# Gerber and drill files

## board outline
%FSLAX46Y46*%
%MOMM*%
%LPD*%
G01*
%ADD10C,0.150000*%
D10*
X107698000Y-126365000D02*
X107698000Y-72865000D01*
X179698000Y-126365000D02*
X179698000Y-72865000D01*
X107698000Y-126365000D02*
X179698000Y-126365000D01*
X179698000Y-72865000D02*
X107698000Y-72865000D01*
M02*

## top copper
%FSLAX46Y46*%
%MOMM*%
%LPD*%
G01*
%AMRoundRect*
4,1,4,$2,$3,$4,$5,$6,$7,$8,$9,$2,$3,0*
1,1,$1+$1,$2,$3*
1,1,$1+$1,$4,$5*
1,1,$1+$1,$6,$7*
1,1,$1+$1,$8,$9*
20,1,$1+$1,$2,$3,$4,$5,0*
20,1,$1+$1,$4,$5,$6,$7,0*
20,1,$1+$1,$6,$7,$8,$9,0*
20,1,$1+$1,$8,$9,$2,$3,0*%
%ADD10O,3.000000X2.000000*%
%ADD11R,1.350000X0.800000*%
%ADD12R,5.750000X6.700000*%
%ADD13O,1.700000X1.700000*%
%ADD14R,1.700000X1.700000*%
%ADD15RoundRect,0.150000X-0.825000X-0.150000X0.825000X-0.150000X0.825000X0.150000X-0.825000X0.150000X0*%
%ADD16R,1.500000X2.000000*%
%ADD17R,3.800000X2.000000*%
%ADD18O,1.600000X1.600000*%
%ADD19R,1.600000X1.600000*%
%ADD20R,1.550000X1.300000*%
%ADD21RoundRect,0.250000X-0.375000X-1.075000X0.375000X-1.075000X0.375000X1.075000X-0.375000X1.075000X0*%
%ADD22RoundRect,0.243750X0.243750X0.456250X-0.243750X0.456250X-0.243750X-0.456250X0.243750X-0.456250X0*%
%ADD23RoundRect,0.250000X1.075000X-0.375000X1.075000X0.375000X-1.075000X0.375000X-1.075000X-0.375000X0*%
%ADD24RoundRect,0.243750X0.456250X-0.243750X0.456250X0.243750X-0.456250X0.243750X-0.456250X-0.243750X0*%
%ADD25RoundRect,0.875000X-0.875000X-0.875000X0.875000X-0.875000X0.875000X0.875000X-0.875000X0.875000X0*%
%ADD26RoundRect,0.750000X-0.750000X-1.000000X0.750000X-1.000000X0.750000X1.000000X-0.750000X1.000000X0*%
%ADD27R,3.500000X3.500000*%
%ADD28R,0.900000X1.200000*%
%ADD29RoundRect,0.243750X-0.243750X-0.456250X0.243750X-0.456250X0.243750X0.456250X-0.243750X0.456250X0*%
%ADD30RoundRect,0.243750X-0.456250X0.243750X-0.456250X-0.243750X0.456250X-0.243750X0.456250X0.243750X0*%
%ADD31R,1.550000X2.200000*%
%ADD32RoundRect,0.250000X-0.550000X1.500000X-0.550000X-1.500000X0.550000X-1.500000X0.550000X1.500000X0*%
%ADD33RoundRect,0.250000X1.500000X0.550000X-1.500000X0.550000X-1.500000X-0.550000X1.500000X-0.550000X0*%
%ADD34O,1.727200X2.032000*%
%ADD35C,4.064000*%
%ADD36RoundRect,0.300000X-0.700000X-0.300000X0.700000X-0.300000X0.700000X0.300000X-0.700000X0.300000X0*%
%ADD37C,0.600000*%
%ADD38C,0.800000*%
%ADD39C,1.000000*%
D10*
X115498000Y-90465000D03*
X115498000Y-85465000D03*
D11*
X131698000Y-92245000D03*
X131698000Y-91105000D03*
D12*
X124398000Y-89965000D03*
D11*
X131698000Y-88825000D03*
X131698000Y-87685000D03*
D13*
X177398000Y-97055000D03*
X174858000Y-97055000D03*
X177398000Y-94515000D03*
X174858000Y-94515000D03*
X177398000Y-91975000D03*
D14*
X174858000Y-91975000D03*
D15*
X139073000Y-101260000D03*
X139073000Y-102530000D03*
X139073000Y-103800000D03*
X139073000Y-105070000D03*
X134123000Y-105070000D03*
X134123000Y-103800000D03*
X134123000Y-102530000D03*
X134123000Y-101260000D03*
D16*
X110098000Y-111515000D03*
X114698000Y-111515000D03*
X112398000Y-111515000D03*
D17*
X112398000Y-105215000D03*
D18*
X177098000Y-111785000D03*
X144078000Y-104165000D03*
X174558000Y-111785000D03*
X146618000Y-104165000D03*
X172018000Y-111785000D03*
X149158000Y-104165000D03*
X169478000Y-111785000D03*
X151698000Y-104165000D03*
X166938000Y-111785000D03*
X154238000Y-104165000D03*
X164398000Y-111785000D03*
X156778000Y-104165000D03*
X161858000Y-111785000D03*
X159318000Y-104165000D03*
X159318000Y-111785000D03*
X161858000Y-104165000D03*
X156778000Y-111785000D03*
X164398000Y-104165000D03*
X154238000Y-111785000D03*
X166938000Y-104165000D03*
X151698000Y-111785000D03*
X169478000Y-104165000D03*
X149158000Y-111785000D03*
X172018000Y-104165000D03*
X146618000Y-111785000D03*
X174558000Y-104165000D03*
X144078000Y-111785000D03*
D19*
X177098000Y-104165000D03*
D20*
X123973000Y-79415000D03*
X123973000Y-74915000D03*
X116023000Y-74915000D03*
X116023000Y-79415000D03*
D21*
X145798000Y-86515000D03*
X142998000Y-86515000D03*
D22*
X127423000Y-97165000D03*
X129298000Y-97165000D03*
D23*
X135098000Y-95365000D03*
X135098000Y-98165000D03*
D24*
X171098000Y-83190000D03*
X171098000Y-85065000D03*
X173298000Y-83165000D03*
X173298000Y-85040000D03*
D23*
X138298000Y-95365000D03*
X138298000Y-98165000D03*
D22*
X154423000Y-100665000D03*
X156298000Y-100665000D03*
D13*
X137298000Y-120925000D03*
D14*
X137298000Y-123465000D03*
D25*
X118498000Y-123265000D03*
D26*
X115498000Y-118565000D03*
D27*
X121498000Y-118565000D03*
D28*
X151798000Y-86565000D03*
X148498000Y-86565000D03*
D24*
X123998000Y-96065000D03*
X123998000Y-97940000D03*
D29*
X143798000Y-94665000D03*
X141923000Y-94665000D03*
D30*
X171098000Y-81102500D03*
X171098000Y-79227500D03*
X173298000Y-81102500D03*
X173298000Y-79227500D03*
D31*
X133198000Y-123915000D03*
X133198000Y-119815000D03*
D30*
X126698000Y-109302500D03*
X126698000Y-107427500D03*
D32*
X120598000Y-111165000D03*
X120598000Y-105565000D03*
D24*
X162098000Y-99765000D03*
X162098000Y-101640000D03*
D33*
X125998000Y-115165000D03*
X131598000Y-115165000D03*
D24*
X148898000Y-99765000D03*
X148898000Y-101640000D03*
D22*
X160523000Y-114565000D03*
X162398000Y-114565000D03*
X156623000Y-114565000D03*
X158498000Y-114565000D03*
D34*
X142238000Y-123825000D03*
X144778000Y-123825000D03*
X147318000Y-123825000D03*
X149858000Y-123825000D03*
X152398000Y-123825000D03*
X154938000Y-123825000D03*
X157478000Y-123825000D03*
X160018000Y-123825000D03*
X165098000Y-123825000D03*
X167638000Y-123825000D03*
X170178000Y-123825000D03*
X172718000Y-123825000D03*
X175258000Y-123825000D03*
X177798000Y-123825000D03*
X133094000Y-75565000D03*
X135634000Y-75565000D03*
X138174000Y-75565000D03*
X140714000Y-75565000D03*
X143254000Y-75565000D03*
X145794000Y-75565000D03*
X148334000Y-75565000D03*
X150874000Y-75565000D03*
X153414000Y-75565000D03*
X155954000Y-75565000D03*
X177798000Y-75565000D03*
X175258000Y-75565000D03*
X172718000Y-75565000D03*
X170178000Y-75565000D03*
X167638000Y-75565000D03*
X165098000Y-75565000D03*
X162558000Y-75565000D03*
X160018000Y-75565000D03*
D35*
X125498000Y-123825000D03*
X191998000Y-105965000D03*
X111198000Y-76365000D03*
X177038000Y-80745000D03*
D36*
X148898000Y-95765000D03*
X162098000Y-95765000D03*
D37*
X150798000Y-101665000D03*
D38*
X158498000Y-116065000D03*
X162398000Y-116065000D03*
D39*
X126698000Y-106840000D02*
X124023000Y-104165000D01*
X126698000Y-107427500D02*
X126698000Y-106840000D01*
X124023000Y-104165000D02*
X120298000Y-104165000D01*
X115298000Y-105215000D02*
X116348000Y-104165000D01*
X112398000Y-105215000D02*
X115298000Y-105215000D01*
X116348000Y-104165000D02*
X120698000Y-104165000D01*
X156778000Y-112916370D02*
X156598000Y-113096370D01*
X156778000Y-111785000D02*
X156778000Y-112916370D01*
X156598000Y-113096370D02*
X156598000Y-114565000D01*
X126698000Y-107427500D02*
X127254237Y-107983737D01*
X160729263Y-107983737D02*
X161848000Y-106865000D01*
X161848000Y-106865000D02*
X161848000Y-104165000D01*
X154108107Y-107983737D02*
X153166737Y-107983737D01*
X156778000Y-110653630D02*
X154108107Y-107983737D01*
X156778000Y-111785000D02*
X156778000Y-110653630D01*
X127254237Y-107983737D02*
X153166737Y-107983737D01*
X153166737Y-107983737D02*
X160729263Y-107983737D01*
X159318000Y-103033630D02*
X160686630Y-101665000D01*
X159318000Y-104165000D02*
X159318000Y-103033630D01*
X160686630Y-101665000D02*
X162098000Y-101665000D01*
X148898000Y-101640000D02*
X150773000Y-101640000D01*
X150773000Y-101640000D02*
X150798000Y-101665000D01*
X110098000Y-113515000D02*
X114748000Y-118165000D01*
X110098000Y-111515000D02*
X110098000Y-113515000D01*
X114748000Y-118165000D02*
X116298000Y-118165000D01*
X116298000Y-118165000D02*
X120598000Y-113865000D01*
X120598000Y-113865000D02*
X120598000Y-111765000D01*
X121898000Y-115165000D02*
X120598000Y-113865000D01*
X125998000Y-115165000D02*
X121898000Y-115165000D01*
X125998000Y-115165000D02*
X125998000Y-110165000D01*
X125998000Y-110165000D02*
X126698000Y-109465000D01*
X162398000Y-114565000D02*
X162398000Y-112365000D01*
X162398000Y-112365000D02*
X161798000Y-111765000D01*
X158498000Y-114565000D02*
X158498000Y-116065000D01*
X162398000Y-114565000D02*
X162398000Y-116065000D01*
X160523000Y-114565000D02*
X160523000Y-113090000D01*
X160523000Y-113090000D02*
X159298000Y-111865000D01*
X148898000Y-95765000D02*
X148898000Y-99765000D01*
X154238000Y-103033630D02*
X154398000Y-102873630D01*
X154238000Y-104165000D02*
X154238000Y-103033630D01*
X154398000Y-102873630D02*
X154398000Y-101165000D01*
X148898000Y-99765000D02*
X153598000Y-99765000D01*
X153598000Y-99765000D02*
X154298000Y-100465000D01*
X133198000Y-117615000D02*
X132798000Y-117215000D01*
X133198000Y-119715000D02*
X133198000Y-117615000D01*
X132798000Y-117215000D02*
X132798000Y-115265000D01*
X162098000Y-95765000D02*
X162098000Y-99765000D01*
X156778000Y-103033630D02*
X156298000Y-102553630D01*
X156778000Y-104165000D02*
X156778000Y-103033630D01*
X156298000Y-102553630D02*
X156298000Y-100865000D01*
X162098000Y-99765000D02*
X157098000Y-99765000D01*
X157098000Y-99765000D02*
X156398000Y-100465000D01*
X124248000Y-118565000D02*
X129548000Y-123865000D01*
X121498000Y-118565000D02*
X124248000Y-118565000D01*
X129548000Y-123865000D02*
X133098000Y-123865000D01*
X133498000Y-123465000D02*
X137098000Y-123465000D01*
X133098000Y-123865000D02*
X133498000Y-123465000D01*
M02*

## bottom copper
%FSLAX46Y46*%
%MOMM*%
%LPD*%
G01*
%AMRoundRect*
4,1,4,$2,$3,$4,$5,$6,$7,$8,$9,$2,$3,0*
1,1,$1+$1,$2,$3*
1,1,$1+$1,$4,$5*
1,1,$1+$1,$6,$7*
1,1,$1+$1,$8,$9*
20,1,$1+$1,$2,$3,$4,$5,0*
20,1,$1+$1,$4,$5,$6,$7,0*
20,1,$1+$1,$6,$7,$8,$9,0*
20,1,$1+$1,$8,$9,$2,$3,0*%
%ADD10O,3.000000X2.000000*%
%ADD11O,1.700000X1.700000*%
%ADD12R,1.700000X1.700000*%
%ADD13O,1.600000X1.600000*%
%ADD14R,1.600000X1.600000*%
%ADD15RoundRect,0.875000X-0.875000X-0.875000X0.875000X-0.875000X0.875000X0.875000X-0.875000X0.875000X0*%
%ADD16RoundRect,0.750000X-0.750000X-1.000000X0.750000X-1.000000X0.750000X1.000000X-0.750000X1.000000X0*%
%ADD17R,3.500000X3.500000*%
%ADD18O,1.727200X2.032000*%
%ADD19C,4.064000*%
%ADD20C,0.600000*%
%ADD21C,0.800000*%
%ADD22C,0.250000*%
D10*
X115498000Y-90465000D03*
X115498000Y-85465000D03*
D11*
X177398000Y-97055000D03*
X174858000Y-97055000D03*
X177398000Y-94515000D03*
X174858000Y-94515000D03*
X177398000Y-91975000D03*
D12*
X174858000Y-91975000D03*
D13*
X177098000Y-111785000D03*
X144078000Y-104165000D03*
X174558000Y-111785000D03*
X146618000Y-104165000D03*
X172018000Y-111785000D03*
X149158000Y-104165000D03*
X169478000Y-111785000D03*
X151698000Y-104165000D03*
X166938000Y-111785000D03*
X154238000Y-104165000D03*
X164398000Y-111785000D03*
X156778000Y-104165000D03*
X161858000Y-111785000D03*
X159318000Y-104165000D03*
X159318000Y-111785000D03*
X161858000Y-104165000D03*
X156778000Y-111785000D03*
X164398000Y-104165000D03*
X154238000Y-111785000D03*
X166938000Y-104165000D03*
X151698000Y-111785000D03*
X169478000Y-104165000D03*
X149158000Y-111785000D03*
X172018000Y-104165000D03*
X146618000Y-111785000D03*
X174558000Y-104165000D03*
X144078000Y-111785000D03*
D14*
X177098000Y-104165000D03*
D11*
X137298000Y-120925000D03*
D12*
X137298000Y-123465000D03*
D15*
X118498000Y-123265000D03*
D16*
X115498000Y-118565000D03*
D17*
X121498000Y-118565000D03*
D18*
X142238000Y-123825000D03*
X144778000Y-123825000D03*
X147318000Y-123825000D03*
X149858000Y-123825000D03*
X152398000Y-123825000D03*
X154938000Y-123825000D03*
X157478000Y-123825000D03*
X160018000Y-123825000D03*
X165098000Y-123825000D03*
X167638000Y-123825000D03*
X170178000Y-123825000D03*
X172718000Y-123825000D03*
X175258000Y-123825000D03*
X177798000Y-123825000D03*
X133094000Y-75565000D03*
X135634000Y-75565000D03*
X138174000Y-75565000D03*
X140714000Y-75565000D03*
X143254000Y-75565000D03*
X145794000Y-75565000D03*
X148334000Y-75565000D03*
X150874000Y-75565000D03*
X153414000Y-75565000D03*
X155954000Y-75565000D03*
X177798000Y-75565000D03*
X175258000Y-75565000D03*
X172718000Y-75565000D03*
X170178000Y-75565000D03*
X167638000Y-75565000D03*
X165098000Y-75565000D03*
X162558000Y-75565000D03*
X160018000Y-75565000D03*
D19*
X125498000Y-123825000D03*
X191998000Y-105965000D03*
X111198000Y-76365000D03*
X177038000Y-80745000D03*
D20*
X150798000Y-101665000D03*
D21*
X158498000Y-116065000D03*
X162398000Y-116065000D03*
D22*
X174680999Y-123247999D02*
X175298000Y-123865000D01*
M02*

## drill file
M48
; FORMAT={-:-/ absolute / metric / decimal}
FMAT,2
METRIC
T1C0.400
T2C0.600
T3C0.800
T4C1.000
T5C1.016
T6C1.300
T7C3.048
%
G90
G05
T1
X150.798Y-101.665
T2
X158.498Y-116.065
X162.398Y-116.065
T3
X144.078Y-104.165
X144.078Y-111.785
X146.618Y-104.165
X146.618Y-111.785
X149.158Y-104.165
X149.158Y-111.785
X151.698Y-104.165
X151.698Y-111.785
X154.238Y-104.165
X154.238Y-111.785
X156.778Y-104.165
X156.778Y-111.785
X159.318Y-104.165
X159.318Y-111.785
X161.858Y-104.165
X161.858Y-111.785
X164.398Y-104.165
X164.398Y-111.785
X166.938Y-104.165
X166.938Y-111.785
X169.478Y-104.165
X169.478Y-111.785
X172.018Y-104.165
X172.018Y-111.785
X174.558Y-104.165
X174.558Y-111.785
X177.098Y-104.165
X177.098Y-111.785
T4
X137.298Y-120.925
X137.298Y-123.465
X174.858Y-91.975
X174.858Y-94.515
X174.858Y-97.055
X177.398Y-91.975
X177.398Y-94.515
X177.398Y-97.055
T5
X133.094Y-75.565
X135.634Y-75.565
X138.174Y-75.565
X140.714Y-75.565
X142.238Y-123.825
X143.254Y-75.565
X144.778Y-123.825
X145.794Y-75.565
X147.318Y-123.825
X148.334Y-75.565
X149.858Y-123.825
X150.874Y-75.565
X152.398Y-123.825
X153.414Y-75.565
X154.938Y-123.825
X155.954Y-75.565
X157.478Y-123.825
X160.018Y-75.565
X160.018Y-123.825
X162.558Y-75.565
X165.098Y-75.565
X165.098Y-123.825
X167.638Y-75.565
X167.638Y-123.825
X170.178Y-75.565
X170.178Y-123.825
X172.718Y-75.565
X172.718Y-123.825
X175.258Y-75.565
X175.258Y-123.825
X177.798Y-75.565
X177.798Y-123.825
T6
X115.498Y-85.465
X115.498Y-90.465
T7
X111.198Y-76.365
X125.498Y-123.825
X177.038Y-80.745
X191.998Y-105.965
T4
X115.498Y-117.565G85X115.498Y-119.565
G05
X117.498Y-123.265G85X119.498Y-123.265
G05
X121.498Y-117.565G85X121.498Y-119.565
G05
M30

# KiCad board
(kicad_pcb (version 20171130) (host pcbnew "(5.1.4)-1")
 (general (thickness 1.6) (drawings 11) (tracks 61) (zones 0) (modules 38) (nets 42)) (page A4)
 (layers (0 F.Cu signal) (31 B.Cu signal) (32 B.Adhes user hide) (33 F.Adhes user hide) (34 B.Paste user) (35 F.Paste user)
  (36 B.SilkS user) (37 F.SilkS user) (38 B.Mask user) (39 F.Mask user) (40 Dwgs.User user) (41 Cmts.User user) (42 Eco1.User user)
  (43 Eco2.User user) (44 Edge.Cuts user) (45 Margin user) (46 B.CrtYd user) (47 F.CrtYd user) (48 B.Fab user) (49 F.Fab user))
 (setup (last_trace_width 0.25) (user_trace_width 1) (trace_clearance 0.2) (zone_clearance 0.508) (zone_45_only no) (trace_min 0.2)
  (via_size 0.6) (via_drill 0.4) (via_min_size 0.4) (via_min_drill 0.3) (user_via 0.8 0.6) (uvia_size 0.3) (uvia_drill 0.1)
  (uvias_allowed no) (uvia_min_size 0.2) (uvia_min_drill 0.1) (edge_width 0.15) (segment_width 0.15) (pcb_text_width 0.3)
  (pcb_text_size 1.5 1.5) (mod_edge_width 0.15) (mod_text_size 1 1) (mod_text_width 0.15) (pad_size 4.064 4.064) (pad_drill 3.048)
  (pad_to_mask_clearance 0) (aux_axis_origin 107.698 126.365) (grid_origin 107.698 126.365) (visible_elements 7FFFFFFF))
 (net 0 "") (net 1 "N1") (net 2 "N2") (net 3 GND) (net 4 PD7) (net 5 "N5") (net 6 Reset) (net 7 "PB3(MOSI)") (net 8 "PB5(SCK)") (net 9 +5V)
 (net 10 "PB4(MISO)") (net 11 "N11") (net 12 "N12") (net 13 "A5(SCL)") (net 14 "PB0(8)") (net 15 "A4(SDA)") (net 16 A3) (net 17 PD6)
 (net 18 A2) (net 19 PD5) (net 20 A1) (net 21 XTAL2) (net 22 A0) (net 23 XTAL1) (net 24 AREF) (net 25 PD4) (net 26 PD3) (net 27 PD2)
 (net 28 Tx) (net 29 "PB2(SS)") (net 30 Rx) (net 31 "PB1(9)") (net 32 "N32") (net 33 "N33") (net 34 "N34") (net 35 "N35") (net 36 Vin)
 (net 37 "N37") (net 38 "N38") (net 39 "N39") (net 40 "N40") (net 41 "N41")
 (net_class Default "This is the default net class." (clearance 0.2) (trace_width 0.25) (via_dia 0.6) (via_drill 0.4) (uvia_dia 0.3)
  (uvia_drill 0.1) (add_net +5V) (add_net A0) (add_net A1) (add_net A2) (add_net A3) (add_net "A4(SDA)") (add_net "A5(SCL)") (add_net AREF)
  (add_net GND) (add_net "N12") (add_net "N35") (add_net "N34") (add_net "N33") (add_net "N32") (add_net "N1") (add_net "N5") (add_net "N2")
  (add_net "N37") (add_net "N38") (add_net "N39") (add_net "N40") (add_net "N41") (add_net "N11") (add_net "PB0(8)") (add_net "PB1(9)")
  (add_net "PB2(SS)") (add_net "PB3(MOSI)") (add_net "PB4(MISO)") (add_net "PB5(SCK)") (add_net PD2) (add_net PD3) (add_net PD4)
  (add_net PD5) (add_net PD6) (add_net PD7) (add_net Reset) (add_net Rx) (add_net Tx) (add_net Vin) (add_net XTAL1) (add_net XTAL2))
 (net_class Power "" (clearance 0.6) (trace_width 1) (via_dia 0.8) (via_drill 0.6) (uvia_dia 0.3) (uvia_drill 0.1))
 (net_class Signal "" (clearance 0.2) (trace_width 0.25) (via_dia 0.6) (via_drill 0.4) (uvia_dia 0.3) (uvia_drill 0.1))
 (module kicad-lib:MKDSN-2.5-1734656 (layer F.Cu) (at 115.498 87.965 90)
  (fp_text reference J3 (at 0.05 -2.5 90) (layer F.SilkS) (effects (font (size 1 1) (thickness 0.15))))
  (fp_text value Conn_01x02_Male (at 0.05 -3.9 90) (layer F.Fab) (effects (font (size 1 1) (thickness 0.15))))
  (pad 1 thru_hole oval (at -2.5 0 90) (size 2 3) (drill 1.3) (layers *.Cu *.Mask) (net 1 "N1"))
  (pad 2 thru_hole oval (at 2.5 0 90) (size 2 3) (drill 1.3) (layers *.Cu *.Mask) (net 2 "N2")))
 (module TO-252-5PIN (layer F.Cu) (at 126.948 89.965 180)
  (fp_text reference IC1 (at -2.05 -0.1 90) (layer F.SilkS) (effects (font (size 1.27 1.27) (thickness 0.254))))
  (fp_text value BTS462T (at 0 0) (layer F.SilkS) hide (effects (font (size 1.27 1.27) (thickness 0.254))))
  (pad 1 smd rect (at -4.75 -2.28 270) (size 0.8 1.35) (layers F.Cu F.Paste F.Mask) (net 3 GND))
  (pad 2 smd rect (at -4.75 -1.14 270) (size 0.8 1.35) (layers F.Cu F.Paste F.Mask) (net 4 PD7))
  (pad 3 smd rect (at 2.55 0 180) (size 5.75 6.7) (layers F.Cu F.Paste F.Mask) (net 1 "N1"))
  (pad 4 smd rect (at -4.75 1.14 270) (size 0.8 1.35) (layers F.Cu F.Paste F.Mask) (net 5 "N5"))
  (pad 5 smd rect (at -4.75 2.28 270) (size 0.8 1.35) (layers F.Cu F.Paste F.Mask) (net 2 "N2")))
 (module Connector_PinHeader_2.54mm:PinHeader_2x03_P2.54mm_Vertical (layer F.Cu) (at 174.858 91.975)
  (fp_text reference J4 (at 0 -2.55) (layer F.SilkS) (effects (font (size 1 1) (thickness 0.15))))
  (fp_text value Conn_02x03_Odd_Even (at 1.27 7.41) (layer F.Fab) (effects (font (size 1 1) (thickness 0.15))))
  (pad 6 thru_hole oval (at 2.54 5.08) (size 1.7 1.7) (drill 1) (layers *.Cu *.Mask) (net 3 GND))
  (pad 5 thru_hole oval (at 0 5.08) (size 1.7 1.7) (drill 1) (layers *.Cu *.Mask) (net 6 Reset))
  (pad 4 thru_hole oval (at 2.54 2.54) (size 1.7 1.7) (drill 1) (layers *.Cu *.Mask) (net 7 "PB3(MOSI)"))
  (pad 3 thru_hole oval (at 0 2.54) (size 1.7 1.7) (drill 1) (layers *.Cu *.Mask) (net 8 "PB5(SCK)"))
  (pad 2 thru_hole oval (at 2.54 0) (size 1.7 1.7) (drill 1) (layers *.Cu *.Mask) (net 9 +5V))
  (pad 1 thru_hole rect (at 0 0) (size 1.7 1.7) (drill 1) (layers *.Cu *.Mask) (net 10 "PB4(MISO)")))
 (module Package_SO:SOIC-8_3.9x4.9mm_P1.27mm (layer F.Cu) (at 136.598 103.165)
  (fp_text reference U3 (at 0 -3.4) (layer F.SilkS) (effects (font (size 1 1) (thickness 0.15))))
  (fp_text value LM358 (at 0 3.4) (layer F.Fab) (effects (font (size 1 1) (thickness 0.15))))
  (pad 8 smd roundrect (at 2.475 -1.905) (size 1.95 0.6) (layers F.Cu F.Paste F.Mask) (roundrect_rratio 0.25) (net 9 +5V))
  (pad 7 smd roundrect (at 2.475 -0.635) (size 1.95 0.6) (layers F.Cu F.Paste F.Mask) (roundrect_rratio 0.25))
  (pad 6 smd roundrect (at 2.475 0.635) (size 1.95 0.6) (layers F.Cu F.Paste F.Mask) (roundrect_rratio 0.25))
  (pad 5 smd roundrect (at 2.475 1.905) (size 1.95 0.6) (layers F.Cu F.Paste F.Mask) (roundrect_rratio 0.25))
  (pad 4 smd roundrect (at -2.475 1.905) (size 1.95 0.6) (layers F.Cu F.Paste F.Mask) (roundrect_rratio 0.25) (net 3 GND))
  (pad 3 smd roundrect (at -2.475 0.635) (size 1.95 0.6) (layers F.Cu F.Paste F.Mask) (roundrect_rratio 0.25) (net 8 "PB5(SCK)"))
  (pad 2 smd roundrect (at -2.475 -0.635) (size 1.95 0.6) (layers F.Cu F.Paste F.Mask) (roundrect_rratio 0.25) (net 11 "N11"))
  (pad 1 smd roundrect (at -2.475 -1.905) (size 1.95 0.6) (layers F.Cu F.Paste F.Mask) (roundrect_rratio 0.25) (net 11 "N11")))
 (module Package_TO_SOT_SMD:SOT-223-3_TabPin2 (layer F.Cu) (at 112.398 108.365 90)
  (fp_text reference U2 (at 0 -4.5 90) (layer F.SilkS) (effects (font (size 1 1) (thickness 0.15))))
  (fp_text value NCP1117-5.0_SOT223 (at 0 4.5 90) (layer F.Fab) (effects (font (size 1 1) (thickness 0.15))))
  (pad 1 smd rect (at -3.15 -2.3 90) (size 2 1.5) (layers F.Cu F.Paste F.Mask) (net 3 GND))
  (pad 3 smd rect (at -3.15 2.3 90) (size 2 1.5) (layers F.Cu F.Paste F.Mask) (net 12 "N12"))
  (pad 2 smd rect (at -3.15 0 90) (size 2 1.5) (layers F.Cu F.Paste F.Mask) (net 9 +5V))
  (pad 2 smd rect (at 3.15 0 90) (size 2 3.8) (layers F.Cu F.Paste F.Mask) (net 9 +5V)))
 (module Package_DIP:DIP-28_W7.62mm (layer F.Cu) (at 177.098 104.165 270)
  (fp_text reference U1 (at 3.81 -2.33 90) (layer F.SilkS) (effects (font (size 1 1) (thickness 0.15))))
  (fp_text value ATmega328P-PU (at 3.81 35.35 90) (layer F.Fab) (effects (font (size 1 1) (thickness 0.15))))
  (pad 28 thru_hole oval (at 7.62 0 270) (size 1.6 1.6) (drill 0.8) (layers *.Cu *.Mask) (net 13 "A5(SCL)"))
  (pad 14 thru_hole oval (at 0 33.02 270) (size 1.6 1.6) (drill 0.8) (layers *.Cu *.Mask) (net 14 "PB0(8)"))
  (pad 27 thru_hole oval (at 7.62 2.54 270) (size 1.6 1.6) (drill 0.8) (layers *.Cu *.Mask) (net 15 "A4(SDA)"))
  (pad 13 thru_hole oval (at 0 30.48 270) (size 1.6 1.6) (drill 0.8) (layers *.Cu *.Mask) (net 4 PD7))
  (pad 26 thru_hole oval (at 7.62 5.08 270) (size 1.6 1.6) (drill 0.8) (layers *.Cu *.Mask) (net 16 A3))
  (pad 12 thru_hole oval (at 0 27.94 270) (size 1.6 1.6) (drill 0.8) (layers *.Cu *.Mask) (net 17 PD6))
  (pad 25 thru_hole oval (at 7.62 7.62 270) (size 1.6 1.6) (drill 0.8) (layers *.Cu *.Mask) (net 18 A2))
  (pad 11 thru_hole oval (at 0 25.4 270) (size 1.6 1.6) (drill 0.8) (layers *.Cu *.Mask) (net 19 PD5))
  (pad 24 thru_hole oval (at 7.62 10.16 270) (size 1.6 1.6) (drill 0.8) (layers *.Cu *.Mask) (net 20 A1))
  (pad 10 thru_hole oval (at 0 22.86 270) (size 1.6 1.6) (drill 0.8) (layers *.Cu *.Mask) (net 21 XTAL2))
  (pad 23 thru_hole oval (at 7.62 12.7 270) (size 1.6 1.6) (drill 0.8) (layers *.Cu *.Mask) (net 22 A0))
  (pad 9 thru_hole oval (at 0 20.32 270) (size 1.6 1.6) (drill 0.8) (layers *.Cu *.Mask) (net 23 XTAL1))
  (pad 22 thru_hole oval (at 7.62 15.24 270) (size 1.6 1.6) (drill 0.8) (layers *.Cu *.Mask) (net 3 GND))
  (pad 8 thru_hole oval (at 0 17.78 270) (size 1.6 1.6) (drill 0.8) (layers *.Cu *.Mask) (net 3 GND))
  (pad 21 thru_hole oval (at 7.62 17.78 270) (size 1.6 1.6) (drill 0.8) (layers *.Cu *.Mask) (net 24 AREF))
  (pad 7 thru_hole oval (at 0 15.24 270) (size 1.6 1.6) (drill 0.8) (layers *.Cu *.Mask) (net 9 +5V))
  (pad 20 thru_hole oval (at 7.62 20.32 270) (size 1.6 1.6) (drill 0.8) (layers *.Cu *.Mask) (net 9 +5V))
  (pad 6 thru_hole oval (at 0 12.7 270) (size 1.6 1.6) (drill 0.8) (layers *.Cu *.Mask) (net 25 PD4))
  (pad 19 thru_hole oval (at 7.62 22.86 270) (size 1.6 1.6) (drill 0.8) (layers *.Cu *.Mask) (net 8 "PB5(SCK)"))
  (pad 5 thru_hole oval (at 0 10.16 270) (size 1.6 1.6) (drill 0.8) (layers *.Cu *.Mask) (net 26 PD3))
  (pad 18 thru_hole oval (at 7.62 25.4 270) (size 1.6 1.6) (drill 0.8) (layers *.Cu *.Mask) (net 10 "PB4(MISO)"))
  (pad 4 thru_hole oval (at 0 7.62 270) (size 1.6 1.6) (drill 0.8) (layers *.Cu *.Mask) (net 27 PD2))
  (pad 17 thru_hole oval (at 7.62 27.94 270) (size 1.6 1.6) (drill 0.8) (layers *.Cu *.Mask) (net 7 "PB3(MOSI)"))
  (pad 3 thru_hole oval (at 0 5.08 270) (size 1.6 1.6) (drill 0.8) (layers *.Cu *.Mask) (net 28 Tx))
  (pad 16 thru_hole oval (at 7.62 30.48 270) (size 1.6 1.6) (drill 0.8) (layers *.Cu *.Mask) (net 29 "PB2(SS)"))
  (pad 2 thru_hole oval (at 0 2.54 270) (size 1.6 1.6) (drill 0.8) (layers *.Cu *.Mask) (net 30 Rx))
  (pad 15 thru_hole oval (at 7.62 33.02 270) (size 1.6 1.6) (drill 0.8) (layers *.Cu *.Mask) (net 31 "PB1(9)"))
  (pad 1 thru_hole rect (at 0 0 270) (size 1.6 1.6) (drill 0.8) (layers *.Cu *.Mask) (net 6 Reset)))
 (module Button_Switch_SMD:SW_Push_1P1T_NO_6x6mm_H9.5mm (layer F.Cu) (at 119.998 77.165)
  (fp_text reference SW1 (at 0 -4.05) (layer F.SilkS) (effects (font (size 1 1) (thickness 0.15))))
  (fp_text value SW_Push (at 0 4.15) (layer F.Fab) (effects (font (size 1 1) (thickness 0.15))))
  (pad 2 smd rect (at 3.975 2.25) (size 1.55 1.3) (layers F.Cu F.Paste F.Mask) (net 3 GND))
  (pad 1 smd rect (at 3.975 -2.25) (size 1.55 1.3) (layers F.Cu F.Paste F.Mask) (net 6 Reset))
  (pad 1 smd rect (at -3.975 -2.25) (size 1.55 1.3) (layers F.Cu F.Paste F.Mask) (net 6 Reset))
  (pad 2 smd rect (at -3.975 2.25) (size 1.55 1.3) (layers F.Cu F.Paste F.Mask) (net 3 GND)))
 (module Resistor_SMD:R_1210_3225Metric (layer F.Cu) (at 144.398 86.515)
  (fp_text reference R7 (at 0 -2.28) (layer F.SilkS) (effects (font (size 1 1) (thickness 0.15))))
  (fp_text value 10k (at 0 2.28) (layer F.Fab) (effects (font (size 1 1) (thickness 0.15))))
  (pad 2 smd roundrect (at 1.4 0) (size 1.25 2.65) (layers F.Cu F.Paste F.Mask) (roundrect_rratio 0.2) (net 6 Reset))
  (pad 1 smd roundrect (at -1.4 0) (size 1.25 2.65) (layers F.Cu F.Paste F.Mask) (roundrect_rratio 0.2) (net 9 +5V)))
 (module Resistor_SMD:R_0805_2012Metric (layer F.Cu) (at 128.3605 97.165 180)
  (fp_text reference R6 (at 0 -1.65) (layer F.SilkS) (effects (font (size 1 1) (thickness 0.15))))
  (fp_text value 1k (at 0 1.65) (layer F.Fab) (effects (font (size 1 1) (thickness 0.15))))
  (pad 2 smd roundrect (at 0.9375 0 180) (size 0.975 1.4) (layers F.Cu F.Paste F.Mask) (roundrect_rratio 0.25) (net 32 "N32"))
  (pad 1 smd roundrect (at -0.9375 0 180) (size 0.975 1.4) (layers F.Cu F.Paste F.Mask) (roundrect_rratio 0.25) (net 11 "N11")))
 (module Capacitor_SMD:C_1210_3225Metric (layer F.Cu) (at 135.098 96.765 90)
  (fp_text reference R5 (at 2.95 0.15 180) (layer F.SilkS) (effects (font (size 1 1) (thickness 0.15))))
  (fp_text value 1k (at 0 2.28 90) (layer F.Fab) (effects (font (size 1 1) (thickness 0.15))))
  (pad 2 smd roundrect (at 1.4 0 90) (size 1.25 2.65) (layers F.Cu F.Paste F.Mask) (roundrect_rratio 0.2) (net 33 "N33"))
  (pad 1 smd roundrect (at -1.4 0 90) (size 1.25 2.65) (layers F.Cu F.Paste F.Mask) (roundrect_rratio 0.2) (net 9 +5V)))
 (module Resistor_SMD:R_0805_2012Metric (layer F.Cu) (at 171.098 84.1275 90)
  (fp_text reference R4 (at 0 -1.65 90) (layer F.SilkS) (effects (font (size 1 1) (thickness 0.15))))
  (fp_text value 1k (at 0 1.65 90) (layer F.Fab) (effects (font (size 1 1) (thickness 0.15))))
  (pad 2 smd roundrect (at 0.9375 0 90) (size 0.975 1.4) (layers F.Cu F.Paste F.Mask) (roundrect_rratio 0.25) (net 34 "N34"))
  (pad 1 smd roundrect (at -0.9375 0 90) (size 0.975 1.4) (layers F.Cu F.Paste F.Mask) (roundrect_rratio 0.25) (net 9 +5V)))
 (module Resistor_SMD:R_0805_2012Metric (layer F.Cu) (at 173.298 84.1025 90)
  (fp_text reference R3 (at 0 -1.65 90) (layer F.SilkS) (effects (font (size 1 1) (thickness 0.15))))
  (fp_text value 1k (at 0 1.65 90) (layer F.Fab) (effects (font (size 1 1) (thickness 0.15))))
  (pad 2 smd roundrect (at 0.9375 0 90) (size 0.975 1.4) (layers F.Cu F.Paste F.Mask) (roundrect_rratio 0.25) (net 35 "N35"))
  (pad 1 smd roundrect (at -0.9375 0 90) (size 0.975 1.4) (layers F.Cu F.Paste F.Mask) (roundrect_rratio 0.25) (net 9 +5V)))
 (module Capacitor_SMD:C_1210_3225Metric (layer F.Cu) (at 138.298 96.765 90)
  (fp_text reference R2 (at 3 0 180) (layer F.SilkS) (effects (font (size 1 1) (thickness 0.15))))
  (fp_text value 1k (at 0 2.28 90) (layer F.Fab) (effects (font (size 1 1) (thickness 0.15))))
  (pad 2 smd roundrect (at 1.4 0 90) (size 1.25 2.65) (layers F.Cu F.Paste F.Mask) (roundrect_rratio 0.2) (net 33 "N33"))
  (pad 1 smd roundrect (at -1.4 0 90) (size 1.25 2.65) (layers F.Cu F.Paste F.Mask) (roundrect_rratio 0.2) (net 9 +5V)))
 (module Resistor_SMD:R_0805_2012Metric (layer F.Cu) (at 155.3605 100.665 180)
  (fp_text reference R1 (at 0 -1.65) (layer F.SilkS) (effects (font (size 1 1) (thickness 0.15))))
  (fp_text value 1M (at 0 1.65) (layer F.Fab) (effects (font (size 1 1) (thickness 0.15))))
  (pad 2 smd roundrect (at 0.9375 0 180) (size 0.975 1.4) (layers F.Cu F.Paste F.Mask) (roundrect_rratio 0.25) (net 21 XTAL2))
  (pad 1 smd roundrect (at -0.9375 0 180) (size 0.975 1.4) (layers F.Cu F.Paste F.Mask) (roundrect_rratio 0.25) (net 23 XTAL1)))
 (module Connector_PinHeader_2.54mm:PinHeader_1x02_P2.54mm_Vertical (layer F.Cu) (at 137.298 123.465 180)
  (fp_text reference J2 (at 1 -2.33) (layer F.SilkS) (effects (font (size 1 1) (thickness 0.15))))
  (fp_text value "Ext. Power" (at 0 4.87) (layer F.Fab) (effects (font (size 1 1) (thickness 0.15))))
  (pad 2 thru_hole oval (at 0 2.54 180) (size 1.7 1.7) (drill 1) (layers *.Cu *.Mask) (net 3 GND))
  (pad 1 thru_hole rect (at 0 0 180) (size 1.7 1.7) (drill 1) (layers *.Cu *.Mask) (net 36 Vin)))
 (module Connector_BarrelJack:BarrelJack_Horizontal (layer F.Cu) (at 121.498 118.565)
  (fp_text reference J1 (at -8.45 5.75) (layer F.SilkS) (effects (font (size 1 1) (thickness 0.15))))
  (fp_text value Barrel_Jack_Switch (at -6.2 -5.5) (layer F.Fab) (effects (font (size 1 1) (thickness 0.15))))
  (pad 3 thru_hole roundrect (at -3 4.7) (size 3.5 3.5) (drill oval 3 1) (layers *.Cu *.Mask) (roundrect_rratio 0.25) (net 3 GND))
  (pad 2 thru_hole roundrect (at -6 0) (size 3 3.5) (drill oval 1 3) (layers *.Cu *.Mask) (roundrect_rratio 0.25) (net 3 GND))
  (pad 1 thru_hole rect (at 0 0) (size 3.5 3.5) (drill oval 1 3) (layers *.Cu *.Mask) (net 36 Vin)))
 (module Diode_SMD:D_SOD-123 (layer F.Cu) (at 150.148 86.565)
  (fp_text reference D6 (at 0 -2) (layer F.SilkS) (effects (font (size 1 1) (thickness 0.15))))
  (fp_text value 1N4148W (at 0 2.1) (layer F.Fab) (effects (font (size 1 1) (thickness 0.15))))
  (pad 2 smd rect (at 1.65 0) (size 0.9 1.2) (layers F.Cu F.Paste F.Mask) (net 6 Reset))
  (pad 1 smd rect (at -1.65 0) (size 0.9 1.2) (layers F.Cu F.Paste F.Mask) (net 9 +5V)))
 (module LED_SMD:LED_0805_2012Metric (layer F.Cu) (at 123.998 97.0025 90)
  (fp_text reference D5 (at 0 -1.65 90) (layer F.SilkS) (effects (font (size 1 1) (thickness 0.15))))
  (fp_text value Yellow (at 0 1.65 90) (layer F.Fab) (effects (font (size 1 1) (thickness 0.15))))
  (pad 2 smd roundrect (at 0.9375 0 90) (size 0.975 1.4) (layers F.Cu F.Paste F.Mask) (roundrect_rratio 0.25) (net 32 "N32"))
  (pad 1 smd roundrect (at -0.9375 0 90) (size 0.975 1.4) (layers F.Cu F.Paste F.Mask) (roundrect_rratio 0.25) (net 3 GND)))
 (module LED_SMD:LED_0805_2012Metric (layer F.Cu) (at 142.8605 94.665)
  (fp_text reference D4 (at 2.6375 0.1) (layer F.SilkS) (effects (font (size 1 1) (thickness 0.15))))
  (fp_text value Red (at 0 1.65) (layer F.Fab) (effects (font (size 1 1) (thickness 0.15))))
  (pad 2 smd roundrect (at 0.9375 0) (size 0.975 1.4) (layers F.Cu F.Paste F.Mask) (roundrect_rratio 0.25) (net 33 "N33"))
  (pad 1 smd roundrect (at -0.9375 0) (size 0.975 1.4) (layers F.Cu F.Paste F.Mask) (roundrect_rratio 0.25) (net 3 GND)))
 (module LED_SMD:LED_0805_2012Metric (layer F.Cu) (at 171.098 80.165 270)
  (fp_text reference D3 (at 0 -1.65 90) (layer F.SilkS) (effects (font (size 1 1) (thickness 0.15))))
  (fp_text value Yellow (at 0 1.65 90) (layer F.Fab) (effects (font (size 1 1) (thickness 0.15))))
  (pad 2 smd roundrect (at 0.9375 0 270) (size 0.975 1.4) (layers F.Cu F.Paste F.Mask) (roundrect_rratio 0.25) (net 34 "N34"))
  (pad 1 smd roundrect (at -0.9375 0 270) (size 0.975 1.4) (layers F.Cu F.Paste F.Mask) (roundrect_rratio 0.25) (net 28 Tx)))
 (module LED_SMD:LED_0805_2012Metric (layer F.Cu) (at 173.298 80.165 270)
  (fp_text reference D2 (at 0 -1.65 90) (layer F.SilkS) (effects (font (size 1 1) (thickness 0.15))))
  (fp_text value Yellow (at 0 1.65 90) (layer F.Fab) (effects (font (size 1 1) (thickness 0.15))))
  (pad 2 smd roundrect (at 0.9375 0 270) (size 0.975 1.4) (layers F.Cu F.Paste F.Mask) (roundrect_rratio 0.25) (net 35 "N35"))
  (pad 1 smd roundrect (at -0.9375 0 270) (size 0.975 1.4) (layers F.Cu F.Paste F.Mask) (roundrect_rratio 0.25) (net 30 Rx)))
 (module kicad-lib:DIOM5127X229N (layer F.Cu) (at 133.198 121.865 270)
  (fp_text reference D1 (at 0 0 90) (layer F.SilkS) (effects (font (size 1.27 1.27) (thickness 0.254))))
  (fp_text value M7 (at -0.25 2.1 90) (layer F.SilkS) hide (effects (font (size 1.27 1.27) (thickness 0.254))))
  (pad 2 smd rect (at 2.05 0) (size 1.55 2.2) (layers F.Cu F.Paste F.Mask) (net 36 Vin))
  (pad 1 smd rect (at -2.05 0) (size 1.55 2.2) (layers F.Cu F.Paste F.Mask) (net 12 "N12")))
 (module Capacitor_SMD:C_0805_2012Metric (layer F.Cu) (at 126.698 108.365 270)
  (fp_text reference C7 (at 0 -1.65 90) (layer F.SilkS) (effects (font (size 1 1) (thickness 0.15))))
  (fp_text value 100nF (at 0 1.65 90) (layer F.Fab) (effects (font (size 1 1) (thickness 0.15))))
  (pad 2 smd roundrect (at 0.9375 0 270) (size 0.975 1.4) (layers F.Cu F.Paste F.Mask) (roundrect_rratio 0.25) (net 3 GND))
  (pad 1 smd roundrect (at -0.9375 0 270) (size 0.975 1.4) (layers F.Cu F.Paste F.Mask) (roundrect_rratio 0.25) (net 9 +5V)))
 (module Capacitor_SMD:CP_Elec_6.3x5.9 (layer F.Cu) (at 120.598 108.365 270)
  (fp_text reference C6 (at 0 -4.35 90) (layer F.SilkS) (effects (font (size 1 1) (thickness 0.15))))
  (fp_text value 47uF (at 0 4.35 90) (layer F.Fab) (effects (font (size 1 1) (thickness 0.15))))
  (pad 2 smd roundrect (at 2.8 0 270) (size 3.5 1.6) (layers F.Cu F.Paste F.Mask) (roundrect_rratio 0.15625) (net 3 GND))
  (pad 1 smd roundrect (at -2.8 0 270) (size 3.5 1.6) (layers F.Cu F.Paste F.Mask) (roundrect_rratio 0.15625) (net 9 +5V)))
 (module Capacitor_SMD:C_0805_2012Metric (layer F.Cu) (at 162.098 100.7025 90)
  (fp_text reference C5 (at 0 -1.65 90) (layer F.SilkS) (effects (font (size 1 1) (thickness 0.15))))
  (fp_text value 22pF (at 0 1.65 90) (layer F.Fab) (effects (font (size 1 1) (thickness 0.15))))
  (pad 2 smd roundrect (at 0.9375 0 90) (size 0.975 1.4) (layers F.Cu F.Paste F.Mask) (roundrect_rratio 0.25) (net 23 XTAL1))
  (pad 1 smd roundrect (at -0.9375 0 90) (size 0.975 1.4) (layers F.Cu F.Paste F.Mask) (roundrect_rratio 0.25) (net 3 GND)))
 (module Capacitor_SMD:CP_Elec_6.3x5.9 (layer F.Cu) (at 128.798 115.165 180)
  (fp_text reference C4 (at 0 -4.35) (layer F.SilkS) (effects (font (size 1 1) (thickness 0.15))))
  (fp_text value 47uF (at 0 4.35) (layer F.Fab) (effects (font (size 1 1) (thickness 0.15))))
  (pad 2 smd roundrect (at 2.8 0 180) (size 3.5 1.6) (layers F.Cu F.Paste F.Mask) (roundrect_rratio 0.15625) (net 3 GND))
  (pad 1 smd roundrect (at -2.8 0 180) (size 3.5 1.6) (layers F.Cu F.Paste F.Mask) (roundrect_rratio 0.15625) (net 12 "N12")))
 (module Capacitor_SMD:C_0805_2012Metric (layer F.Cu) (at 148.898 100.7025 90)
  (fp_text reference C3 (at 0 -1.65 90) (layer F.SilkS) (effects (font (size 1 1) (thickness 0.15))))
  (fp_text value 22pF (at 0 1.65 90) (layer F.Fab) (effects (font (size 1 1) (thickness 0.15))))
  (pad 2 smd roundrect (at 0.9375 0 90) (size 0.975 1.4) (layers F.Cu F.Paste F.Mask) (roundrect_rratio 0.25) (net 21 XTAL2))
  (pad 1 smd roundrect (at -0.9375 0 90) (size 0.975 1.4) (layers F.Cu F.Paste F.Mask) (roundrect_rratio 0.25) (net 3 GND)))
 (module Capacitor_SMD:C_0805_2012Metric (layer F.Cu) (at 161.4605 114.565 180)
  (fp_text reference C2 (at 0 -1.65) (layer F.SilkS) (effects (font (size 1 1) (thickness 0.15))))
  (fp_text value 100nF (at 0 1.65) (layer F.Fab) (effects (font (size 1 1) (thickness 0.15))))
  (pad 2 smd roundrect (at 0.9375 0 180) (size 0.975 1.4) (layers F.Cu F.Paste F.Mask) (roundrect_rratio 0.25) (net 24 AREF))
  (pad 1 smd roundrect (at -0.9375 0 180) (size 0.975 1.4) (layers F.Cu F.Paste F.Mask) (roundrect_rratio 0.25) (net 3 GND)))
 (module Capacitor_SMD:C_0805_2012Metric (layer F.Cu) (at 157.5605 114.565 180)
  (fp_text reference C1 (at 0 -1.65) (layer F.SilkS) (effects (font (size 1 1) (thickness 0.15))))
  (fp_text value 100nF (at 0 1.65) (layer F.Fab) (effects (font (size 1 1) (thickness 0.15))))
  (pad 2 smd roundrect (at 0.9375 0 180) (size 0.975 1.4) (layers F.Cu F.Paste F.Mask) (roundrect_rratio 0.25) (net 9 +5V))
  (pad 1 smd roundrect (at -0.9375 0 180) (size 0.975 1.4) (layers F.Cu F.Paste F.Mask) (roundrect_rratio 0.25) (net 3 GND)))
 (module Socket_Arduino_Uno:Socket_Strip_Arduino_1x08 (layer F.Cu) (at 142.238 123.825)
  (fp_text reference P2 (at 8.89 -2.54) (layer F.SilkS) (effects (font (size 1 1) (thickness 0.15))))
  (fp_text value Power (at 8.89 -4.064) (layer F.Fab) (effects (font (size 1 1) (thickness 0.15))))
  (pad 1 thru_hole oval (at 0 0) (size 1.7272 2.032) (drill 1.016) (layers *.Cu *.Mask F.SilkS) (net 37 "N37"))
  (pad 2 thru_hole oval (at 2.54 0) (size 1.7272 2.032) (drill 1.016) (layers *.Cu *.Mask F.SilkS) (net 9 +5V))
  (pad 3 thru_hole oval (at 5.08 0) (size 1.7272 2.032) (drill 1.016) (layers *.Cu *.Mask F.SilkS) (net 6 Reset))
  (pad 4 thru_hole oval (at 7.62 0) (size 1.7272 2.032) (drill 1.016) (layers *.Cu *.Mask F.SilkS) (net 9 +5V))
  (pad 5 thru_hole oval (at 10.16 0) (size 1.7272 2.032) (drill 1.016) (layers *.Cu *.Mask F.SilkS) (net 9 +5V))
  (pad 6 thru_hole oval (at 12.7 0) (size 1.7272 2.032) (drill 1.016) (layers *.Cu *.Mask F.SilkS) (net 3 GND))
  (pad 7 thru_hole oval (at 15.24 0) (size 1.7272 2.032) (drill 1.016) (layers *.Cu *.Mask F.SilkS) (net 3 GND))
  (pad 8 thru_hole oval (at 17.78 0) (size 1.7272 2.032) (drill 1.016) (layers *.Cu *.Mask F.SilkS) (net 36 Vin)))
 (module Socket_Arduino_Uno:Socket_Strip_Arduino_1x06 (layer F.Cu) (at 165.098 123.825)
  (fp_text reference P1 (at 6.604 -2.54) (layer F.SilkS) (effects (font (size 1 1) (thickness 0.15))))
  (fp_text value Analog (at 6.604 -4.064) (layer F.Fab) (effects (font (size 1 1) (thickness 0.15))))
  (pad 1 thru_hole oval (at 0 0) (size 1.7272 2.032) (drill 1.016) (layers *.Cu *.Mask F.SilkS) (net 22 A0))
  (pad 2 thru_hole oval (at 2.54 0) (size 1.7272 2.032) (drill 1.016) (layers *.Cu *.Mask F.SilkS) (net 20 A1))
  (pad 3 thru_hole oval (at 5.08 0) (size 1.7272 2.032) (drill 1.016) (layers *.Cu *.Mask F.SilkS) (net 18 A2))
  (pad 4 thru_hole oval (at 7.62 0) (size 1.7272 2.032) (drill 1.016) (layers *.Cu *.Mask F.SilkS) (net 16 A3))
  (pad 5 thru_hole oval (at 10.16 0) (size 1.7272 2.032) (drill 1.016) (layers *.Cu *.Mask F.SilkS) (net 15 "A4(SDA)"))
  (pad 6 thru_hole oval (at 12.7 0) (size 1.7272 2.032) (drill 1.016) (layers *.Cu *.Mask F.SilkS) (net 13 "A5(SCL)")))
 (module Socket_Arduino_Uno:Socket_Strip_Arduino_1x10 (layer F.Cu) (at 133.094 75.565)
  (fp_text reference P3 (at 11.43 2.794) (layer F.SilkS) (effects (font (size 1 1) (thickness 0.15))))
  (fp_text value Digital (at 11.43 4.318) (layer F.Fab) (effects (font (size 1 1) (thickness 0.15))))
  (pad 1 thru_hole oval (at 0 0) (size 1.7272 2.032) (drill 1.016) (layers *.Cu *.Mask F.SilkS) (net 14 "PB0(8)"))
  (pad 2 thru_hole oval (at 2.54 0) (size 1.7272 2.032) (drill 1.016) (layers *.Cu *.Mask F.SilkS) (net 31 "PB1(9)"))
  (pad 3 thru_hole oval (at 5.08 0) (size 1.7272 2.032) (drill 1.016) (layers *.Cu *.Mask F.SilkS) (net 29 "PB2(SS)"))
  (pad 4 thru_hole oval (at 7.62 0) (size 1.7272 2.032) (drill 1.016) (layers *.Cu *.Mask F.SilkS) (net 7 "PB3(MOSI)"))
  (pad 5 thru_hole oval (at 10.16 0) (size 1.7272 2.032) (drill 1.016) (layers *.Cu *.Mask F.SilkS) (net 10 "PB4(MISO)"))
  (pad 6 thru_hole oval (at 12.7 0) (size 1.7272 2.032) (drill 1.016) (layers *.Cu *.Mask F.SilkS) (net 8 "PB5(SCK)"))
  (pad 7 thru_hole oval (at 15.24 0) (size 1.7272 2.032) (drill 1.016) (layers *.Cu *.Mask F.SilkS) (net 3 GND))
  (pad 8 thru_hole oval (at 17.78 0) (size 1.7272 2.032) (drill 1.016) (layers *.Cu *.Mask F.SilkS) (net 24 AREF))
  (pad 9 thru_hole oval (at 20.32 0) (size 1.7272 2.032) (drill 1.016) (layers *.Cu *.Mask F.SilkS) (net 15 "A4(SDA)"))
  (pad 10 thru_hole oval (at 22.86 0) (size 1.7272 2.032) (drill 1.016) (layers *.Cu *.Mask F.SilkS) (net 13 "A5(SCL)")))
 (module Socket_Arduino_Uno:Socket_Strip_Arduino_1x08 (layer F.Cu) (at 177.798 75.565 180)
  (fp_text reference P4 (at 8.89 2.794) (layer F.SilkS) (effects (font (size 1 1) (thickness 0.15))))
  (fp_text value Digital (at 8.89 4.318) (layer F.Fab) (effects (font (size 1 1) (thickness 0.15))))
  (pad 1 thru_hole oval (at 0 0 180) (size 1.7272 2.032) (drill 1.016) (layers *.Cu *.Mask F.SilkS) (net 30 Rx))
  (pad 2 thru_hole oval (at 2.54 0 180) (size 1.7272 2.032) (drill 1.016) (layers *.Cu *.Mask F.SilkS) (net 28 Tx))
  (pad 3 thru_hole oval (at 5.08 0 180) (size 1.7272 2.032) (drill 1.016) (layers *.Cu *.Mask F.SilkS) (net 27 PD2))
  (pad 4 thru_hole oval (at 7.62 0 180) (size 1.7272 2.032) (drill 1.016) (layers *.Cu *.Mask F.SilkS) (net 26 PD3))
  (pad 5 thru_hole oval (at 10.16 0 180) (size 1.7272 2.032) (drill 1.016) (layers *.Cu *.Mask F.SilkS) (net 25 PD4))
  (pad 6 thru_hole oval (at 12.7 0 180) (size 1.7272 2.032) (drill 1.016) (layers *.Cu *.Mask F.SilkS) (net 19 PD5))
  (pad 7 thru_hole oval (at 15.24 0 180) (size 1.7272 2.032) (drill 1.016) (layers *.Cu *.Mask F.SilkS) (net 17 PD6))
  (pad 8 thru_hole oval (at 17.78 0 180) (size 1.7272 2.032) (drill 1.016) (layers *.Cu *.Mask F.SilkS) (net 4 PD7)))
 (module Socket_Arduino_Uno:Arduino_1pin (layer F.Cu) (at 125.498 123.825)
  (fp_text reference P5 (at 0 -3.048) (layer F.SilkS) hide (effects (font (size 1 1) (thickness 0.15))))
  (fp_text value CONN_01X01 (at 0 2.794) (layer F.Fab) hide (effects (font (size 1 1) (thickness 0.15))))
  (pad 1 thru_hole circle (at 0 0) (size 4.064 4.064) (drill 3.048) (layers *.Cu *.Mask F.SilkS) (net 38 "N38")))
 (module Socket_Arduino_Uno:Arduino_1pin (layer F.Cu) (at 191.998 105.965)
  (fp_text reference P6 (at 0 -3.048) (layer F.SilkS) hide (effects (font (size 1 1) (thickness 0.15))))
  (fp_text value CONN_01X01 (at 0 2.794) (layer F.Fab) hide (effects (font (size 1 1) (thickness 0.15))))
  (pad 1 thru_hole circle (at 0 0) (size 4.064 4.064) (drill 3.048) (layers *.Cu *.Mask F.SilkS) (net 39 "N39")))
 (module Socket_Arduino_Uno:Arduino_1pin (layer F.Cu) (at 111.198 76.365)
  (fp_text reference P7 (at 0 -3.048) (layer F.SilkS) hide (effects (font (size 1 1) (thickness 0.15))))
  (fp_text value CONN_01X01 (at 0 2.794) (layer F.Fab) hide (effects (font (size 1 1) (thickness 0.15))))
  (pad 1 thru_hole circle (at 0 0) (size 4.064 4.064) (drill 3.048) (layers *.Cu *.Mask F.SilkS) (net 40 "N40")))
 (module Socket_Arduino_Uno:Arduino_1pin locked (layer F.Cu) (at 177.038 80.745)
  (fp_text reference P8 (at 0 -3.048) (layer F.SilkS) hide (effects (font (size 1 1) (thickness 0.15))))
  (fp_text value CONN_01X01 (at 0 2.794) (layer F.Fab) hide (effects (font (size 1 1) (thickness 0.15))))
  (pad 1 thru_hole circle (at 0 0) (size 4.064 4.064) (drill 3.048) (layers *.Cu *.Mask F.SilkS) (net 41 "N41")))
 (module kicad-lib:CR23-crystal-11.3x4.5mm (layer F.Cu) (at 155.498 95.765)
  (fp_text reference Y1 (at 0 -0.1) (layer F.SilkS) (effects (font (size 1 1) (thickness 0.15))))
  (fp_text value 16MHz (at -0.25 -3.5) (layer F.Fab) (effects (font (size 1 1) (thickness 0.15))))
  (pad 1 smd roundrect (at -6.6 0) (size 2 1.2) (layers F.Cu F.Paste F.Mask) (roundrect_rratio 0.25) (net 21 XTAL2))
  (pad 2 smd roundrect (at 6.6 0) (size 2 1.2) (layers F.Cu F.Paste F.Mask) (roundrect_rratio 0.25) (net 23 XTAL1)))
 (gr_line (start 107.698 126.365) (end 107.698 72.865) (layer Edge.Cuts) (width 0.15))
 (gr_line (start 179.698 126.365) (end 179.698 72.865) (angle 90) (layer Edge.Cuts) (width 0.15))
 (gr_line (start 107.698 126.365) (end 179.698 126.365) (angle 90) (layer Edge.Cuts) (width 0.15))
 (gr_line (start 179.698 72.865) (end 107.698 72.865) (angle 90) (layer Edge.Cuts) (width 0.15))
 (segment (start 126.698 106.84) (end 124.023 104.165) (width 1) (layer F.Cu) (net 9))
 (segment (start 126.698 107.4275) (end 126.698 106.84) (width 1) (layer F.Cu) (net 9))
 (segment (start 124.023 104.165) (end 120.298 104.165) (width 1) (layer F.Cu) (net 9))
 (segment (start 115.298 105.215) (end 116.348 104.165) (width 1) (layer F.Cu) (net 9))
 (segment (start 112.398 105.215) (end 115.298 105.215) (width 1) (layer F.Cu) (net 9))
 (segment (start 116.348 104.165) (end 120.698 104.165) (width 1) (layer F.Cu) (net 9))
 (segment (start 156.778 112.91637) (end 156.598 113.09637) (width 1) (layer F.Cu) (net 9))
 (segment (start 156.778 111.785) (end 156.778 112.91637) (width 1) (layer F.Cu) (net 9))
 (segment (start 156.598 113.09637) (end 156.598 114.565) (width 1) (layer F.Cu) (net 9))
 (segment (start 126.698 107.4275) (end 127.254237 107.983737) (width 1) (layer F.Cu) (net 9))
 (segment (start 160.729263 107.983737) (end 161.848 106.865) (width 1) (layer F.Cu) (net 9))
 (segment (start 161.848 106.865) (end 161.848 104.165) (width 1) (layer F.Cu) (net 9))
 (segment (start 154.108107 107.983737) (end 153.166737 107.983737) (width 1) (layer F.Cu) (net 9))
 (segment (start 156.778 110.65363) (end 154.108107 107.983737) (width 1) (layer F.Cu) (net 9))
 (segment (start 156.778 111.785) (end 156.778 110.65363) (width 1) (layer F.Cu) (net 9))
 (segment (start 127.254237 107.983737) (end 153.166737 107.983737) (width 1) (layer F.Cu) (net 9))
 (segment (start 153.166737 107.983737) (end 160.729263 107.983737) (width 1) (layer F.Cu) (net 9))
 (segment (start 159.318 103.03363) (end 160.68663 101.665) (width 1) (layer F.Cu) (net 3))
 (segment (start 159.318 104.165) (end 159.318 103.03363) (width 1) (layer F.Cu) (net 3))
 (segment (start 160.68663 101.665) (end 162.098 101.665) (width 1) (layer F.Cu) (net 3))
 (via (at 150.798 101.665) (size 0.6) (drill 0.4) (layers F.Cu B.Cu) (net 3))
 (segment (start 148.898 101.64) (end 150.773 101.64) (width 1) (layer F.Cu) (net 3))
 (segment (start 150.773 101.64) (end 150.798 101.665) (width 1) (layer F.Cu) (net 3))
 (segment (start 110.098 113.515) (end 114.748 118.165) (width 1) (layer F.Cu) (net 3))
 (segment (start 110.098 111.515) (end 110.098 113.515) (width 1) (layer F.Cu) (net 3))
 (segment (start 114.748 118.165) (end 116.298 118.165) (width 1) (layer F.Cu) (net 3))
 (segment (start 116.298 118.165) (end 120.598 113.865) (width 1) (layer F.Cu) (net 3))
 (segment (start 120.598 113.865) (end 120.598 111.765) (width 1) (layer F.Cu) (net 3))
 (segment (start 121.898 115.165) (end 120.598 113.865) (width 1) (layer F.Cu) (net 3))
 (segment (start 125.998 115.165) (end 121.898 115.165) (width 1) (layer F.Cu) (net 3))
 (segment (start 125.998 115.165) (end 125.998 110.165) (width 1) (layer F.Cu) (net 3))
 (segment (start 125.998 110.165) (end 126.698 109.465) (width 1) (layer F.Cu) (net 3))
 (segment (start 162.398 114.565) (end 162.398 112.365) (width 1) (layer F.Cu) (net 3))
 (segment (start 162.398 112.365) (end 161.798 111.765) (width 1) (layer F.Cu) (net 3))
 (via (at 158.498 116.065) (size 0.8) (drill 0.6) (layers F.Cu B.Cu) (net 3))
 (segment (start 158.498 114.565) (end 158.498 116.065) (width 1) (layer F.Cu) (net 3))
 (via (at 162.398 116.065) (size 0.8) (drill 0.6) (layers F.Cu B.Cu) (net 3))
 (segment (start 162.398 114.565) (end 162.398 116.065) (width 1) (layer F.Cu) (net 3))
 (segment (start 160.523 114.565) (end 160.523 113.09) (width 1) (layer F.Cu) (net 24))
 (segment (start 160.523 113.09) (end 159.298 111.865) (width 1) (layer F.Cu) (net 24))
 (segment (start 148.898 95.765) (end 148.898 99.765) (width 1) (layer F.Cu) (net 21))
 (segment (start 154.238 103.03363) (end 154.398 102.87363) (width 1) (layer F.Cu) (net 21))
 (segment (start 154.238 104.165) (end 154.238 103.03363) (width 1) (layer F.Cu) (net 21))
 (segment (start 154.398 102.87363) (end 154.398 101.165) (width 1) (layer F.Cu) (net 21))
 (segment (start 148.898 99.765) (end 153.598 99.765) (width 1) (layer F.Cu) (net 21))
 (segment (start 153.598 99.765) (end 154.298 100.465) (width 1) (layer F.Cu) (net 21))
 (segment (start 133.198 117.615) (end 132.798 117.215) (width 1) (layer F.Cu) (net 12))
 (segment (start 133.198 119.715) (end 133.198 117.615) (width 1) (layer F.Cu) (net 12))
 (segment (start 132.798 117.215) (end 132.798 115.265) (width 1) (layer F.Cu) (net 12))
 (segment (start 162.098 95.765) (end 162.098 99.765) (width 1) (layer F.Cu) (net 23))
 (segment (start 156.778 103.03363) (end 156.298 102.55363) (width 1) (layer F.Cu) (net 23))
 (segment (start 156.778 104.165) (end 156.778 103.03363) (width 1) (layer F.Cu) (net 23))
 (segment (start 156.298 102.55363) (end 156.298 100.865) (width 1) (layer F.Cu) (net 23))
 (segment (start 162.098 99.765) (end 157.098 99.765) (width 1) (layer F.Cu) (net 23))
 (segment (start 157.098 99.765) (end 156.398 100.465) (width 1) (layer F.Cu) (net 23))
 (segment (start 124.248 118.565) (end 129.548 123.865) (width 1) (layer F.Cu) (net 36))
 (segment (start 121.498 118.565) (end 124.248 118.565) (width 1) (layer F.Cu) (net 36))
 (segment (start 129.548 123.865) (end 133.098 123.865) (width 1) (layer F.Cu) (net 36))
 (segment (start 133.498 123.465) (end 137.098 123.465) (width 1) (layer F.Cu) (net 36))
 (segment (start 133.098 123.865) (end 133.498 123.465) (width 1) (layer F.Cu) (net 36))
 (segment (start 174.680999 123.247999) (end 175.298 123.865) (width 0.25) (layer B.Cu) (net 15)))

